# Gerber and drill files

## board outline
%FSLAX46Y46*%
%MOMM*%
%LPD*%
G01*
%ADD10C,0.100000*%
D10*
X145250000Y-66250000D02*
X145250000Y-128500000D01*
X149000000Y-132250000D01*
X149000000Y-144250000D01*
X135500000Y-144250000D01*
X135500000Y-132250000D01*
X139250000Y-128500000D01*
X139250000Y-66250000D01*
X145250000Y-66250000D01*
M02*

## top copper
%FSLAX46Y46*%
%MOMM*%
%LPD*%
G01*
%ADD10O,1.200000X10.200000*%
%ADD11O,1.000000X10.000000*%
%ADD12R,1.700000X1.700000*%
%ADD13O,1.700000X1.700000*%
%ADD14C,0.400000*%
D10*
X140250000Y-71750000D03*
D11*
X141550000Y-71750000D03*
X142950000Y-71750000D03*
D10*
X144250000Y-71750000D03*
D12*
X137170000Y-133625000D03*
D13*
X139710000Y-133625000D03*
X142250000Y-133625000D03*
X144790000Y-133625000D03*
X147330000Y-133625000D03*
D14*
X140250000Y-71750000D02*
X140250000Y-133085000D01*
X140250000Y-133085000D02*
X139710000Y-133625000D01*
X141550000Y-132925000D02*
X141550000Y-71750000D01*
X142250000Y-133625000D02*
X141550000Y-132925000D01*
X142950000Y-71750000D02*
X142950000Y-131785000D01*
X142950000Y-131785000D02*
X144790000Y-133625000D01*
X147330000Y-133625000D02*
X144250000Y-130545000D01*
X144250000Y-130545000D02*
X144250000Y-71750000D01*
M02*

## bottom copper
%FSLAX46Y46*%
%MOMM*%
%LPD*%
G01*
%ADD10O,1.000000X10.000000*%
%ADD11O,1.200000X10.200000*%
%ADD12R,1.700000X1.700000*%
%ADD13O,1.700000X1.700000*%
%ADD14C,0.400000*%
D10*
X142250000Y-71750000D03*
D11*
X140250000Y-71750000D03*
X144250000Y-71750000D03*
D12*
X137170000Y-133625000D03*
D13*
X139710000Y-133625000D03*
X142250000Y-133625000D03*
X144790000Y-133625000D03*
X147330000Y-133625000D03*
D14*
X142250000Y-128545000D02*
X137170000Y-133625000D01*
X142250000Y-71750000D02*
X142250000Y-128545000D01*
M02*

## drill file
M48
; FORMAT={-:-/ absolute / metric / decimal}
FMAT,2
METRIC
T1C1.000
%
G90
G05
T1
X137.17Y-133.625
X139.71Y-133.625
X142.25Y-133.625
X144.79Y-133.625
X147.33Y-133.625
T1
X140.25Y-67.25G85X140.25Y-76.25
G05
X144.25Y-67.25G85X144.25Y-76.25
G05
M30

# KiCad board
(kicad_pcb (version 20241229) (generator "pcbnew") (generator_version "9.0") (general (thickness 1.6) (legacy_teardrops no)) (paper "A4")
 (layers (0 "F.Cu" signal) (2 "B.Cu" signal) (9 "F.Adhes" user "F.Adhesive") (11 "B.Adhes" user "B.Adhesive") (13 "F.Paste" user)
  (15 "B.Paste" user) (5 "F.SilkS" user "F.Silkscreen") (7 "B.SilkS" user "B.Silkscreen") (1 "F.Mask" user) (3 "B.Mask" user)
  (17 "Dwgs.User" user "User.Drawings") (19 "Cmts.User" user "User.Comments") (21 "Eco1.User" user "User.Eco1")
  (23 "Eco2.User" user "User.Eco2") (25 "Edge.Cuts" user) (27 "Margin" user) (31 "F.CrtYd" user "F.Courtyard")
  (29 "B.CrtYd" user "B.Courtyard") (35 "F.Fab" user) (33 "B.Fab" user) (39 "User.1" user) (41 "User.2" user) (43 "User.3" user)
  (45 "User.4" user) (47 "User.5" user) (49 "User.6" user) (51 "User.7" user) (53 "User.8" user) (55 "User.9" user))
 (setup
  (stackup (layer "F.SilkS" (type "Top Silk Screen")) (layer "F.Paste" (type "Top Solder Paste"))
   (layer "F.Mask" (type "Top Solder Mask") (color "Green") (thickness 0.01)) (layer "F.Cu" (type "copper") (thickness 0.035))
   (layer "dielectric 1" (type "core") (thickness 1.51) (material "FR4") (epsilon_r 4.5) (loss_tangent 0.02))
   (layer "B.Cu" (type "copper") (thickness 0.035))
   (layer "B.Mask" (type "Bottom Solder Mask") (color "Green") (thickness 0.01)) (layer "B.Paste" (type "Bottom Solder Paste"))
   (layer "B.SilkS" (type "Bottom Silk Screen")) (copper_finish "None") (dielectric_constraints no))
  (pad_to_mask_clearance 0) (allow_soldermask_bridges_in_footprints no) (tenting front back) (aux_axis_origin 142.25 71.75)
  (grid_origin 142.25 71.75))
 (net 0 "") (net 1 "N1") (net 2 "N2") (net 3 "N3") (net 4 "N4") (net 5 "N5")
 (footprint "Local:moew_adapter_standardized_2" (layer "F.Cu") (at 142.25 71.75)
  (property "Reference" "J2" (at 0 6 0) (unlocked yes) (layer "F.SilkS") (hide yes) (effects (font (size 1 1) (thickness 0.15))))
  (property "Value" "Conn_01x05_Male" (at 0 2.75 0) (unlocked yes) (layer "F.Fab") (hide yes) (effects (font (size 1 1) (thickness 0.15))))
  (pad "1" smd oval (at 0 0) (size 1 10) (layers "B.Cu" "B.Mask") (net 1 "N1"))
  (pad "2" thru_hole oval (at -2 0) (size 1.2 10.2) (drill oval 1 10) (layers "*.Cu" "B.Mask") (remove_unused_layers no) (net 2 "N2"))
  (pad "3" smd oval (at -0.7 0) (size 1 10) (layers "F.Cu" "F.Mask") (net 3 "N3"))
  (pad "4" smd oval (at 0.7 0) (size 1 10) (layers "F.Cu" "F.Mask") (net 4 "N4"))
  (pad "5" thru_hole oval (at 2 0) (size 1.2 10.2) (drill oval 1 10) (layers "*.Cu" "B.Mask") (remove_unused_layers no) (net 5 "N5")))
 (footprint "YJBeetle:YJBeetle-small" (layer "F.Cu") (at 142.25 136 180)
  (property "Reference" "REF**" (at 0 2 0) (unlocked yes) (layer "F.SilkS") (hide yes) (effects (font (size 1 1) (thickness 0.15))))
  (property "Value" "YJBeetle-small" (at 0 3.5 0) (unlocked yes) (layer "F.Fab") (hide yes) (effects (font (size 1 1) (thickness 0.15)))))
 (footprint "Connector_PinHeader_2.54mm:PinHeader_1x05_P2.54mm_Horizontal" (layer "B.Cu") (at 137.17 133.625 -90)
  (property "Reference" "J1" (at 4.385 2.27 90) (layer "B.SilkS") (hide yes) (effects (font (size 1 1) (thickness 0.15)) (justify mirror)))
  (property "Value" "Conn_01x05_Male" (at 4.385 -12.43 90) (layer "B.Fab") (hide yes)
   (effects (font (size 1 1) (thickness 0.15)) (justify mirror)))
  (pad "1" thru_hole rect (at 0 0 270) (size 1.7 1.7) (drill 1) (layers "*.Cu" "*.Mask") (remove_unused_layers no) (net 1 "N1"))
  (pad "2" thru_hole oval (at 0 -2.54 270) (size 1.7 1.7) (drill 1) (layers "*.Cu" "*.Mask") (remove_unused_layers no) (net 2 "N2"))
  (pad "3" thru_hole oval (at 0 -5.08 270) (size 1.7 1.7) (drill 1) (layers "*.Cu" "*.Mask") (remove_unused_layers no) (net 3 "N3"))
  (pad "4" thru_hole oval (at 0 -7.62 270) (size 1.7 1.7) (drill 1) (layers "*.Cu" "*.Mask") (remove_unused_layers no) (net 4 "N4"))
  (pad "5" thru_hole oval (at 0 -10.16 270) (size 1.7 1.7) (drill 1) (layers "*.Cu" "*.Mask") (remove_unused_layers no) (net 5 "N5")))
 (gr_poly
  (pts (xy 145.25 66.25) (xy 145.25 128.5) (xy 149 132.25) (xy 149 144.25) (xy 135.5 144.25) (xy 135.5 132.25) (xy 139.25 128.5)
   (xy 139.25 66.25))
  (stroke (width 0.1) (type solid)) (fill no) (layer "Edge.Cuts"))
 (segment (start 142.25 128.545) (end 137.17 133.625) (width 0.4) (layer "B.Cu") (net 1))
 (segment (start 142.25 71.75) (end 142.25 128.545) (width 0.4) (layer "B.Cu") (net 1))
 (segment (start 140.25 71.75) (end 140.25 133.085) (width 0.4) (layer "F.Cu") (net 2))
 (segment (start 140.25 133.085) (end 139.71 133.625) (width 0.4) (layer "F.Cu") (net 2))
 (segment (start 141.55 132.925) (end 141.55 71.75) (width 0.4) (layer "F.Cu") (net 3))
 (segment (start 142.25 133.625) (end 141.55 132.925) (width 0.4) (layer "F.Cu") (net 3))
 (segment (start 142.95 71.75) (end 142.95 131.785) (width 0.4) (layer "F.Cu") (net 4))
 (segment (start 142.95 131.785) (end 144.79 133.625) (width 0.4) (layer "F.Cu") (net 4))
 (segment (start 147.33 133.625) (end 144.25 130.545) (width 0.4) (layer "F.Cu") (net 5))
 (segment (start 144.25 130.545) (end 144.25 71.75) (width 0.4) (layer "F.Cu") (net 5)))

